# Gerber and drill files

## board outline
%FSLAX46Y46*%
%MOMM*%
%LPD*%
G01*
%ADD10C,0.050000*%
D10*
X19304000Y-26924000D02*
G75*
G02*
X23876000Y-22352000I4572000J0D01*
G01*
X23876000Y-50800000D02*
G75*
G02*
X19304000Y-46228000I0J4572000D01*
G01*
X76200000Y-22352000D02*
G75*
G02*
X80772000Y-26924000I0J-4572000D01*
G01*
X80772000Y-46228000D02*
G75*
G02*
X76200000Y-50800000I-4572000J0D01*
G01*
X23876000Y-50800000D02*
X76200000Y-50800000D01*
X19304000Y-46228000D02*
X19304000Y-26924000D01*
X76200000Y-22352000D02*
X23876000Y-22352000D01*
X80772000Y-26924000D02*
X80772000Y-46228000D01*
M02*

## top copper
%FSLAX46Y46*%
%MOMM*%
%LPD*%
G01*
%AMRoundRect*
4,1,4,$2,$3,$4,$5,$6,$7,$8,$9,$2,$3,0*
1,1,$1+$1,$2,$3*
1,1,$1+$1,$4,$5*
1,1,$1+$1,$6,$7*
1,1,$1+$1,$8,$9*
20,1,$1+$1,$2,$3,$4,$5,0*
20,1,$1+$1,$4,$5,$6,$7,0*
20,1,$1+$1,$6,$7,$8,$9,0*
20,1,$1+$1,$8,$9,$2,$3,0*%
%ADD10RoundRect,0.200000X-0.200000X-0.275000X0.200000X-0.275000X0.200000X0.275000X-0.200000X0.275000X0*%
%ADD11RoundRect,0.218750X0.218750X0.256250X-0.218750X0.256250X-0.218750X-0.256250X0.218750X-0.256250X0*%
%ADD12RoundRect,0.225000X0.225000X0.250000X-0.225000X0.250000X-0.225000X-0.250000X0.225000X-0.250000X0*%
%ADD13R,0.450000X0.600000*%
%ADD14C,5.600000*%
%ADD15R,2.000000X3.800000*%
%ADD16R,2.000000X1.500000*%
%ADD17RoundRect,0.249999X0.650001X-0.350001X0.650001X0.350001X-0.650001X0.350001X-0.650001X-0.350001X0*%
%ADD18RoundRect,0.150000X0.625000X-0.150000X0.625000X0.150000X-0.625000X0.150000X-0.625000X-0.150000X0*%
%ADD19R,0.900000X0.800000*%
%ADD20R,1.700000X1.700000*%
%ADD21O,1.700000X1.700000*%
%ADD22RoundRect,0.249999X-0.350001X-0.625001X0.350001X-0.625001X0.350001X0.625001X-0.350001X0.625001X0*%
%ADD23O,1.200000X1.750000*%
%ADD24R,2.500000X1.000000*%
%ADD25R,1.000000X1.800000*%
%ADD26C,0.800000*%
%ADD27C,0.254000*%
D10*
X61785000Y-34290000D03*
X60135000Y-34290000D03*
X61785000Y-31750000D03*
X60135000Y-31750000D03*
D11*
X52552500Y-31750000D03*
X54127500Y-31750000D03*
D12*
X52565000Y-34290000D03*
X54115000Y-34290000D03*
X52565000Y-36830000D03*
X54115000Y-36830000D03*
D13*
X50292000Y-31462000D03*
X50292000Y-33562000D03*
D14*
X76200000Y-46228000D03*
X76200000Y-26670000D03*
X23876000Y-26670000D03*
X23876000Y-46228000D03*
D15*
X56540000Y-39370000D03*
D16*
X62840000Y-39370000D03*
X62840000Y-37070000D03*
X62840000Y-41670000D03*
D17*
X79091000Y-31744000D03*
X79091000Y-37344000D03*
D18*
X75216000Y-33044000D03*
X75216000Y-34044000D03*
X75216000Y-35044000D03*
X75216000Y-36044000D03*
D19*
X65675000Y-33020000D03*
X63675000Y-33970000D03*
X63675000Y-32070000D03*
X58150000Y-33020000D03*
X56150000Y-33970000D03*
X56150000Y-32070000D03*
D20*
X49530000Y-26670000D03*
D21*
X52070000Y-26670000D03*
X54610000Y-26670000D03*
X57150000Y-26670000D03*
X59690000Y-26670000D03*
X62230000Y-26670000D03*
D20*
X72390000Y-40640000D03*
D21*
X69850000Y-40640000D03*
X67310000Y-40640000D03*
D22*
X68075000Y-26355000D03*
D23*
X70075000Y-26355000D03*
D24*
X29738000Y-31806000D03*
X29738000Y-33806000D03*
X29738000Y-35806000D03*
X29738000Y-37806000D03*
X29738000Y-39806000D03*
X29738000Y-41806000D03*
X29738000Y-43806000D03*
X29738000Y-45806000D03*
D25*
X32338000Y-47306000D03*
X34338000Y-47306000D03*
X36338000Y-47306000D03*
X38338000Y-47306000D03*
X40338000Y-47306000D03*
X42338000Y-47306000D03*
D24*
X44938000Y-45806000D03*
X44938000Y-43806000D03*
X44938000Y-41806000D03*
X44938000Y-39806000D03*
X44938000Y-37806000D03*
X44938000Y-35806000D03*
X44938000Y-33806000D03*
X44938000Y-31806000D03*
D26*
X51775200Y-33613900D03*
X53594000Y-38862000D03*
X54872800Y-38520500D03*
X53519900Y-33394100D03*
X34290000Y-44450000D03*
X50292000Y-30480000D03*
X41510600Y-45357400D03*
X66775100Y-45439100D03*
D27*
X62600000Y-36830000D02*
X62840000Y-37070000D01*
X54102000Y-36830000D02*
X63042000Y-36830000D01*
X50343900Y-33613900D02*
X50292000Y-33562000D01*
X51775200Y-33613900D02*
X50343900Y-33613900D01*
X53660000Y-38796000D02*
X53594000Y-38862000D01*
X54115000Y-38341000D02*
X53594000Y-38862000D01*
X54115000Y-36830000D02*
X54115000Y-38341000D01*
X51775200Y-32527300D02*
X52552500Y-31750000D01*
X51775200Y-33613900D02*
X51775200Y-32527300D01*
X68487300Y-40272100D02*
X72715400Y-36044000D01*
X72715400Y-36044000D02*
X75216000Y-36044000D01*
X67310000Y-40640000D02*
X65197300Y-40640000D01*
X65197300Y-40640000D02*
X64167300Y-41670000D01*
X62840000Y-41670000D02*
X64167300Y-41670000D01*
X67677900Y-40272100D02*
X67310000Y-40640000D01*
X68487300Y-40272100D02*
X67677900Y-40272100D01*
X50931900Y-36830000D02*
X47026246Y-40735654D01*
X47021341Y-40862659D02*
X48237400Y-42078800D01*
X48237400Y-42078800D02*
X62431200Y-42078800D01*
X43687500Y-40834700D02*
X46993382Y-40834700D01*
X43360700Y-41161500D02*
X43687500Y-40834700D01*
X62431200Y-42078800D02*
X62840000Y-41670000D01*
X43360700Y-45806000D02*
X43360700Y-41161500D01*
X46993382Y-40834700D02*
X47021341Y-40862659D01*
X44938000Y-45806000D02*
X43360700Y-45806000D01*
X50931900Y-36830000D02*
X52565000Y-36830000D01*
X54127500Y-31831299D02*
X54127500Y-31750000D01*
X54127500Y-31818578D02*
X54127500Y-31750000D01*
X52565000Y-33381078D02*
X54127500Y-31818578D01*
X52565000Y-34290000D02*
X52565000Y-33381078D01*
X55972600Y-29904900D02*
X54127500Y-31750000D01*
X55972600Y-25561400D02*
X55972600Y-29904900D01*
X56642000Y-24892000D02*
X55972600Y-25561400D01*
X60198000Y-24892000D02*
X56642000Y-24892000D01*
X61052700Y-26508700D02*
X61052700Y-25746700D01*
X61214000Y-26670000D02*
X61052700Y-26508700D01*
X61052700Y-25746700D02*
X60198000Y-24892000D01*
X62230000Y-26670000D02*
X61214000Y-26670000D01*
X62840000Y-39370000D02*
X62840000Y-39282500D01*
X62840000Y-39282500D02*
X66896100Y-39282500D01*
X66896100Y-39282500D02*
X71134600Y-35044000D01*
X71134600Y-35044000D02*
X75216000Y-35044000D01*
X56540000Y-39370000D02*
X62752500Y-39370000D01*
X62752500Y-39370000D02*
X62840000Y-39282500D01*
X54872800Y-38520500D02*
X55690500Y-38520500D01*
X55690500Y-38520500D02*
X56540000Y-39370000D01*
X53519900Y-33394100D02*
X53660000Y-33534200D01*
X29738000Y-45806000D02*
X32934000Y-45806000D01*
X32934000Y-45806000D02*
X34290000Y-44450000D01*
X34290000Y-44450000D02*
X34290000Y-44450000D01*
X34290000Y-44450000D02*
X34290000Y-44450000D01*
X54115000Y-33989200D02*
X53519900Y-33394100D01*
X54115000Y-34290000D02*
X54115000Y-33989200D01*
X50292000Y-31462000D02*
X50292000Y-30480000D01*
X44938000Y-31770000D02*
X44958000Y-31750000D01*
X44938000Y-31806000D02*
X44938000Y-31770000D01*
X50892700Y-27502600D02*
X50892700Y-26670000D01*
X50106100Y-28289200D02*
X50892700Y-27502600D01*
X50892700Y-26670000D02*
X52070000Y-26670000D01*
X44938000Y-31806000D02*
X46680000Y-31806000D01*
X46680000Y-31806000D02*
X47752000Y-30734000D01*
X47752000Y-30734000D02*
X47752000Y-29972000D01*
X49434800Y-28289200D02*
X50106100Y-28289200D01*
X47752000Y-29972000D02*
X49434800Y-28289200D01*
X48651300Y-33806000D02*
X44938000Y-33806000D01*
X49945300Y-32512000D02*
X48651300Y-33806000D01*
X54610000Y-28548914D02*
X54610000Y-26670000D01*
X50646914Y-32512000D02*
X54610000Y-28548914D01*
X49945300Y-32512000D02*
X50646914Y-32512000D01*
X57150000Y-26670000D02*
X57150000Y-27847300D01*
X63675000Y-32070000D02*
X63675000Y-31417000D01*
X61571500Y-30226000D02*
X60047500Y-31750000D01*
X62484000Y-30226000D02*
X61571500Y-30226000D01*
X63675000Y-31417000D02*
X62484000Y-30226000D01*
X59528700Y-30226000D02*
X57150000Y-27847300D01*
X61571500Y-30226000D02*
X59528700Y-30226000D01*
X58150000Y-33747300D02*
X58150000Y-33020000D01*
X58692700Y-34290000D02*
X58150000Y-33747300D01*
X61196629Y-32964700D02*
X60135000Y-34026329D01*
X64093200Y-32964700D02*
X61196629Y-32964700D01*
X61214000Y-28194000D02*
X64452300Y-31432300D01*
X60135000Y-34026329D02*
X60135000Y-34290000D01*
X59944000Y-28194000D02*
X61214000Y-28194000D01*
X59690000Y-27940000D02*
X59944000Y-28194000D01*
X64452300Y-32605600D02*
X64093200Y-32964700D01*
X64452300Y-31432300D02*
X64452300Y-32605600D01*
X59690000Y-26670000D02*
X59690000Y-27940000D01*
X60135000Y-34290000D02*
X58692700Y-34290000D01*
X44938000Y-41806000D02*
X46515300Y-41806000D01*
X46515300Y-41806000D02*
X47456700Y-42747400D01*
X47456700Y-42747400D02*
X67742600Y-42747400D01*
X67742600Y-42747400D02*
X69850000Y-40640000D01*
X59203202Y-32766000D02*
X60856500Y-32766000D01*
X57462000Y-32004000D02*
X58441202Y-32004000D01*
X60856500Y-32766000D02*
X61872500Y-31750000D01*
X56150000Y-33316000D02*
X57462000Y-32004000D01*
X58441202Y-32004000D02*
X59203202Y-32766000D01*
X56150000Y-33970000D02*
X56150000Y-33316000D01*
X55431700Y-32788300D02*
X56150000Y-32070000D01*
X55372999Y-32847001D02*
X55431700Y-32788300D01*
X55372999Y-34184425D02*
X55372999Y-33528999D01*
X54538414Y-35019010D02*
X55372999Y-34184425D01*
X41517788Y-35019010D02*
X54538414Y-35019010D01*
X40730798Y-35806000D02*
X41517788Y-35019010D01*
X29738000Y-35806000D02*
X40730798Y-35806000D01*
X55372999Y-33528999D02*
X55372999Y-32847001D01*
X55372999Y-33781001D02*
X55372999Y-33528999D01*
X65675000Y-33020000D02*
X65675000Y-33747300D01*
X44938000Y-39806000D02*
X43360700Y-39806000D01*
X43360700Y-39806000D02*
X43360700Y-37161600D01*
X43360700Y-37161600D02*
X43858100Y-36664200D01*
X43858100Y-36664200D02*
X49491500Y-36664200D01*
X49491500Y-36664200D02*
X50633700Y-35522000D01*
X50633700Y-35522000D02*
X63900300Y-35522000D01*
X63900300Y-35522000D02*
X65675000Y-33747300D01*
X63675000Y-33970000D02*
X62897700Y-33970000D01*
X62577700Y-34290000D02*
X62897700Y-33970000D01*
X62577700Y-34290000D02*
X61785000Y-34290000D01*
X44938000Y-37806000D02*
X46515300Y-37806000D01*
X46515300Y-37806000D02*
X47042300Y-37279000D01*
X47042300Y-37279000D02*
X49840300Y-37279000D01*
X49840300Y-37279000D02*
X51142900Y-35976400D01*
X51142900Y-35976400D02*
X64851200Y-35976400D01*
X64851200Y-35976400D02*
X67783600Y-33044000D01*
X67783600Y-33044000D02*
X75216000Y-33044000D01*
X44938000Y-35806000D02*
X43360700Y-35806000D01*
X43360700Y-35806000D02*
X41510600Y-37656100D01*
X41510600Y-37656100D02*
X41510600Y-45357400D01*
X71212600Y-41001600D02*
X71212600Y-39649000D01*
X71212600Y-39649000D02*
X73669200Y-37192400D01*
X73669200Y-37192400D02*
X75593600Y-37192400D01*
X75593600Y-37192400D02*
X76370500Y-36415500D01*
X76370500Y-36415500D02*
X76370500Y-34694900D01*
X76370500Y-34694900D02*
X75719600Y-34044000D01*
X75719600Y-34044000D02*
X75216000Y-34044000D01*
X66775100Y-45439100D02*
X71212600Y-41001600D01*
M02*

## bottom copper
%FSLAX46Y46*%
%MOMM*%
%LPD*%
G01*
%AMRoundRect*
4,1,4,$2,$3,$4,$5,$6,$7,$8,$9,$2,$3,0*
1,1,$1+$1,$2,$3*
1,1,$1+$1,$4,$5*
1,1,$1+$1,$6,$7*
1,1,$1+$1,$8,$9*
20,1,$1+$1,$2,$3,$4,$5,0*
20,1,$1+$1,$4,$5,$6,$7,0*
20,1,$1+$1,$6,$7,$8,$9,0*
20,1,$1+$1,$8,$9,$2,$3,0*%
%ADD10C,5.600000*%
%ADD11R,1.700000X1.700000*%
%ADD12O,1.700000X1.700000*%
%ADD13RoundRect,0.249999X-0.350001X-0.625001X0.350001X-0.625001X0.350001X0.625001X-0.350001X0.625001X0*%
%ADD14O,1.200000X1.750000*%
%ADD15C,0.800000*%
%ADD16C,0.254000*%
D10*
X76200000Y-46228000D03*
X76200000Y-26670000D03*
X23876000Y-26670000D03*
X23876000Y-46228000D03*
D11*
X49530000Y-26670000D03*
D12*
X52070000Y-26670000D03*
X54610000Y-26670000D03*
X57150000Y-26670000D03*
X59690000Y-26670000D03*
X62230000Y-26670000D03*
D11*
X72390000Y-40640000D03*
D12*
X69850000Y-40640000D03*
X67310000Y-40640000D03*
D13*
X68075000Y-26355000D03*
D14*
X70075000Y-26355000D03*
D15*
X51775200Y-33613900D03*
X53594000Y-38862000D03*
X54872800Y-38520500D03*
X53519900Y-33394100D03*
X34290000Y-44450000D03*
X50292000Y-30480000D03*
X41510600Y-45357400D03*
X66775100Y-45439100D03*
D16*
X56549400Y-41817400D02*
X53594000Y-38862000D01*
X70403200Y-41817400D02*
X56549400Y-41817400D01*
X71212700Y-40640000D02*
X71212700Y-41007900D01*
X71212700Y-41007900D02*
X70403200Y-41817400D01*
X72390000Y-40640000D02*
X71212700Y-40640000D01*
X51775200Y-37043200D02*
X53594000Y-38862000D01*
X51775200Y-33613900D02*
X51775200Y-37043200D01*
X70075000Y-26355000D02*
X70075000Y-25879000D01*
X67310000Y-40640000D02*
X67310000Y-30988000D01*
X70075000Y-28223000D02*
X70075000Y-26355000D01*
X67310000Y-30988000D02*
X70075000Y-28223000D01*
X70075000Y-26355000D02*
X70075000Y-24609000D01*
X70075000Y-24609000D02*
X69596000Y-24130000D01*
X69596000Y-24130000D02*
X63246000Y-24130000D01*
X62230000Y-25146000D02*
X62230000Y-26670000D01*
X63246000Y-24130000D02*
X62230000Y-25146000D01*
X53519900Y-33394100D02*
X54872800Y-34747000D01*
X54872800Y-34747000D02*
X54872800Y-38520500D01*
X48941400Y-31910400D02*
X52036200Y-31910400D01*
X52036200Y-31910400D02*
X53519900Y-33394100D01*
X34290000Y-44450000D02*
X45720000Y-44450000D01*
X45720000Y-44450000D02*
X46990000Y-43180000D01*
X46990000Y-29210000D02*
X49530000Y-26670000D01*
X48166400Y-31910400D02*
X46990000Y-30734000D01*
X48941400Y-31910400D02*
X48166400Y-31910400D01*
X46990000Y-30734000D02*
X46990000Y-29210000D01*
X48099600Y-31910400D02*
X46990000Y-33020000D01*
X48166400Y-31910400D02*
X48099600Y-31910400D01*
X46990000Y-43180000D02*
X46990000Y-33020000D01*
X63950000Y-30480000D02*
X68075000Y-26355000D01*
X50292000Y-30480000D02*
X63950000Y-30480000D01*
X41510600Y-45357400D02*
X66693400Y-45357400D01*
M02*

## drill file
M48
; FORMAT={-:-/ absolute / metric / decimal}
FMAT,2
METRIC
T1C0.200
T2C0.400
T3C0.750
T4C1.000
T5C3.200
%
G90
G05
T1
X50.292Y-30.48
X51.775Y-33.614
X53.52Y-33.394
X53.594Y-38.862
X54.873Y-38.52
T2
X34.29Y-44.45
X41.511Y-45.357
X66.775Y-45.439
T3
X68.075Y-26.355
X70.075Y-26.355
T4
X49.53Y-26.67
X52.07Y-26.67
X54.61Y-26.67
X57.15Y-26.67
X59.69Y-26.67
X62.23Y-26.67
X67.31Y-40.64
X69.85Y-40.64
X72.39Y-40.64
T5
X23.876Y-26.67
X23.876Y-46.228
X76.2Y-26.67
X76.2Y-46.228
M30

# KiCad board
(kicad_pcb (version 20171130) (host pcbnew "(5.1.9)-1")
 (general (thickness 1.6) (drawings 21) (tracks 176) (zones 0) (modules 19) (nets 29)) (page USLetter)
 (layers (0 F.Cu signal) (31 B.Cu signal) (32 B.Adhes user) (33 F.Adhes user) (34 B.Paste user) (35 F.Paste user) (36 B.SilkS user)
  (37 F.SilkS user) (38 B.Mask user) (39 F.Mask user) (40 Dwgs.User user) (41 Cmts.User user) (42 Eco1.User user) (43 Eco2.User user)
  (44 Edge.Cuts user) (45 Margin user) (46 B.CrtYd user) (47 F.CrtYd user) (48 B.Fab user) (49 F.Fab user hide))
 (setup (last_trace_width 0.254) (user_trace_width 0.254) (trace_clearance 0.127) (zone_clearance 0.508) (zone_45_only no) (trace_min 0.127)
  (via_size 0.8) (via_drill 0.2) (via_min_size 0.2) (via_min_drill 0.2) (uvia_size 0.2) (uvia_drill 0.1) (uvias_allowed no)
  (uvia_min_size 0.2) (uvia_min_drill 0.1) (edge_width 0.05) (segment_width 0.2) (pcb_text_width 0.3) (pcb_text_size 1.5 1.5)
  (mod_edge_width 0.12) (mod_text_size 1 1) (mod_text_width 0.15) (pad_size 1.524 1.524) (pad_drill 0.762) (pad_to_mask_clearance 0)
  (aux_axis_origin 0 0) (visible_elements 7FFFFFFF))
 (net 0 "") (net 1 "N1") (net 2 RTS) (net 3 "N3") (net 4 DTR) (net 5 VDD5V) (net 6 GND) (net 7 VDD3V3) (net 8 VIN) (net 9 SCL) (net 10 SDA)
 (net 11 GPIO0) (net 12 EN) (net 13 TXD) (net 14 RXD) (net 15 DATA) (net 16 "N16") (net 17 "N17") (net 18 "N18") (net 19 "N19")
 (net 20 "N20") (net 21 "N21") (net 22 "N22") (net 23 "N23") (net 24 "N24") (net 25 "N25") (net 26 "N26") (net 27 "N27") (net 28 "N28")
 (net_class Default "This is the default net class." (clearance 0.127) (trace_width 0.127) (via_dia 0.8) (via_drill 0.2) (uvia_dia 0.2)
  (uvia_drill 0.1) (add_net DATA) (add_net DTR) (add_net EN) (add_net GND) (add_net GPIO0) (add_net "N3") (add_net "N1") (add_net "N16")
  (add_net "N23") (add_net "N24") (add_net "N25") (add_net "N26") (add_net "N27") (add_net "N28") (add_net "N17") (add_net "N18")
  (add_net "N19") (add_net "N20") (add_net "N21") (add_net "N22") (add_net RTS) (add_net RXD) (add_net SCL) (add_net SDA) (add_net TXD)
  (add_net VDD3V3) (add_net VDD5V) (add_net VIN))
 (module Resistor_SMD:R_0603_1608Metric (layer F.Cu) (at 60.96 34.29)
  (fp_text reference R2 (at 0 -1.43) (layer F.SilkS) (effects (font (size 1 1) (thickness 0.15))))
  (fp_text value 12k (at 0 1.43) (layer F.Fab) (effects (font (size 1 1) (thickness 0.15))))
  (pad 2 smd roundrect (at 0.825 0) (size 0.8 0.95) (layers F.Cu F.Paste F.Mask) (roundrect_rratio 0.25) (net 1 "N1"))
  (pad 1 smd roundrect (at -0.825 0) (size 0.8 0.95) (layers F.Cu F.Paste F.Mask) (roundrect_rratio 0.25) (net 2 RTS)))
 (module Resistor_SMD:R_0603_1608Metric (layer F.Cu) (at 60.96 31.75)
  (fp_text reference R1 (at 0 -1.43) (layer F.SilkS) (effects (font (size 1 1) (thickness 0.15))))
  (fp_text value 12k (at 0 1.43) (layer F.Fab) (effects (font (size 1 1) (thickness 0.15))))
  (pad 2 smd roundrect (at 0.825 0) (size 0.8 0.95) (layers F.Cu F.Paste F.Mask) (roundrect_rratio 0.25) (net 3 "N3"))
  (pad 1 smd roundrect (at -0.825 0) (size 0.8 0.95) (layers F.Cu F.Paste F.Mask) (roundrect_rratio 0.25) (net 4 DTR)))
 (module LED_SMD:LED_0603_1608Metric (layer F.Cu) (at 53.34 31.75 180)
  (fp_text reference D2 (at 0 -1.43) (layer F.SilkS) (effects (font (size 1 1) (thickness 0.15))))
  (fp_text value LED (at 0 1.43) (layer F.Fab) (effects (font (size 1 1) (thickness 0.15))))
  (pad 2 smd roundrect (at 0.7875 0 180) (size 0.875 0.95) (layers F.Cu F.Paste F.Mask) (roundrect_rratio 0.25) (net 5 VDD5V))
  (pad 1 smd roundrect (at -0.7875 0 180) (size 0.875 0.95) (layers F.Cu F.Paste F.Mask) (roundrect_rratio 0.25) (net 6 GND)))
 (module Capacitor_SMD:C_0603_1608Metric (layer F.Cu) (at 53.34 34.29 180)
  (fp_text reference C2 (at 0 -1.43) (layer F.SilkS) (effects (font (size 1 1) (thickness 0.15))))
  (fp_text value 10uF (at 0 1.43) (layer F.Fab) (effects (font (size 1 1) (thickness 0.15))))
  (pad 2 smd roundrect (at 0.775 0 180) (size 0.9 0.95) (layers F.Cu F.Paste F.Mask) (roundrect_rratio 0.25) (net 6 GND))
  (pad 1 smd roundrect (at -0.775 0 180) (size 0.9 0.95) (layers F.Cu F.Paste F.Mask) (roundrect_rratio 0.25) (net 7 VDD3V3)))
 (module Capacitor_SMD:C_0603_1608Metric (layer F.Cu) (at 53.34 36.83 180)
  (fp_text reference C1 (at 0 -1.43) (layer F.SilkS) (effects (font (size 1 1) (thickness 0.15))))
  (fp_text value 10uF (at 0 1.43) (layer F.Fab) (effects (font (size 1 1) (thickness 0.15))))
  (pad 2 smd roundrect (at 0.775 0 180) (size 0.9 0.95) (layers F.Cu F.Paste F.Mask) (roundrect_rratio 0.25) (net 6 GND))
  (pad 1 smd roundrect (at -0.775 0 180) (size 0.9 0.95) (layers F.Cu F.Paste F.Mask) (roundrect_rratio 0.25) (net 5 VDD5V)))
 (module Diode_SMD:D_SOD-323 (layer F.Cu) (at 50.292 32.512 90)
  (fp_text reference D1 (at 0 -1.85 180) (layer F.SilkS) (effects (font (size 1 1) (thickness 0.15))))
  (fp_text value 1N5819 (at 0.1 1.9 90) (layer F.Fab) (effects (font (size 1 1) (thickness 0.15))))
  (pad 2 smd rect (at 1.05 0 90) (size 0.6 0.45) (layers F.Cu F.Paste F.Mask) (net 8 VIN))
  (pad 1 smd rect (at -1.05 0 90) (size 0.6 0.45) (layers F.Cu F.Paste F.Mask) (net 5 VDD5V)))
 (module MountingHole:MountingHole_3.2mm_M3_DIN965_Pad (layer F.Cu) (at 76.2 46.228)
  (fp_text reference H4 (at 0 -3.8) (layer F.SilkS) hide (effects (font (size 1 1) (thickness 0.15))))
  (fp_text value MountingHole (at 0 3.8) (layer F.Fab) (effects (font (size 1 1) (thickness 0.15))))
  (pad 1 thru_hole circle (at 0 0) (size 5.6 5.6) (drill 3.2) (layers *.Cu *.Mask)))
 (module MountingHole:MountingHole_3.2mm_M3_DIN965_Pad (layer F.Cu) (at 76.2 26.67)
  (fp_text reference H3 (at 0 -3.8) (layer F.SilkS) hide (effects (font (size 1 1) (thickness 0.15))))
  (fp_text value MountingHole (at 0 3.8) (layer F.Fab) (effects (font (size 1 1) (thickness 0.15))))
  (pad 1 thru_hole circle (at 0 0) (size 5.6 5.6) (drill 3.2) (layers *.Cu *.Mask)))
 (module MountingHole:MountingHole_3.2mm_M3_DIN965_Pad (layer F.Cu) (at 23.876 26.67)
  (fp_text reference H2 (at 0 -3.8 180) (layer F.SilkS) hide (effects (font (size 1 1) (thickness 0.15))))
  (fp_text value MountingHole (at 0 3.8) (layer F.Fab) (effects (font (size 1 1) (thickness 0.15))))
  (pad 1 thru_hole circle (at 0 0) (size 5.6 5.6) (drill 3.2) (layers *.Cu *.Mask)))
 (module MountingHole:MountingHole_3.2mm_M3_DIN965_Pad (layer F.Cu) (at 23.876 46.228)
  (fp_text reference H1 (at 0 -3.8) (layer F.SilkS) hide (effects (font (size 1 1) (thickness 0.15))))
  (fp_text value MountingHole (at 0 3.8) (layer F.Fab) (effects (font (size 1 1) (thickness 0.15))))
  (pad 1 thru_hole circle (at 0 0) (size 5.6 5.6) (drill 3.2) (layers *.Cu *.Mask)))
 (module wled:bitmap (layer F.Cu) (at 70.612 34.29)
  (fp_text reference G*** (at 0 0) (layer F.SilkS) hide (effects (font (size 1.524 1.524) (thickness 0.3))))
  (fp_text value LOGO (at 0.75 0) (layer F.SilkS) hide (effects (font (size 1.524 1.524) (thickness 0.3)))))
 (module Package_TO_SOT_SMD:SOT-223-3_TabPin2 (layer F.Cu) (at 59.69 39.37 180)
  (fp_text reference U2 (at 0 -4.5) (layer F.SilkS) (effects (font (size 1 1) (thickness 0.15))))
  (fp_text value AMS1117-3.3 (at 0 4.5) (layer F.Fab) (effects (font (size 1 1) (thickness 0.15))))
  (pad 2 smd rect (at 3.15 0 180) (size 2 3.8) (layers F.Cu F.Paste F.Mask) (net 7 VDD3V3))
  (pad 2 smd rect (at -3.15 0 180) (size 2 1.5) (layers F.Cu F.Paste F.Mask) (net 7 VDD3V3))
  (pad 3 smd rect (at -3.15 2.3 180) (size 2 1.5) (layers F.Cu F.Paste F.Mask) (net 5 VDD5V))
  (pad 1 smd rect (at -3.15 -2.3 180) (size 2 1.5) (layers F.Cu F.Paste F.Mask) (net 6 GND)))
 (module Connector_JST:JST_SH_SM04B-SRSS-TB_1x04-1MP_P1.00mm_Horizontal (layer F.Cu) (at 77.216 34.544 90)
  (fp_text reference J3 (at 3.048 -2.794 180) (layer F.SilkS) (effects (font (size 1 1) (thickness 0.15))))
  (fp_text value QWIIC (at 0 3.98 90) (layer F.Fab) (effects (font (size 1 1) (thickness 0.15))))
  (pad MP smd roundrect (at 2.8 1.875 90) (size 1.2 1.8) (layers F.Cu F.Paste F.Mask) (roundrect_rratio 0.2083325))
  (pad MP smd roundrect (at -2.8 1.875 90) (size 1.2 1.8) (layers F.Cu F.Paste F.Mask) (roundrect_rratio 0.2083325))
  (pad 4 smd roundrect (at 1.5 -2 90) (size 0.6 1.55) (layers F.Cu F.Paste F.Mask) (roundrect_rratio 0.25) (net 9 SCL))
  (pad 3 smd roundrect (at 0.5 -2 90) (size 0.6 1.55) (layers F.Cu F.Paste F.Mask) (roundrect_rratio 0.25) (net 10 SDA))
  (pad 2 smd roundrect (at -0.5 -2 90) (size 0.6 1.55) (layers F.Cu F.Paste F.Mask) (roundrect_rratio 0.25) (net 7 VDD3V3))
  (pad 1 smd roundrect (at -1.5 -2 90) (size 0.6 1.55) (layers F.Cu F.Paste F.Mask) (roundrect_rratio 0.25) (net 6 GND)))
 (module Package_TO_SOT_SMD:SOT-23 (layer F.Cu) (at 64.675 33.02)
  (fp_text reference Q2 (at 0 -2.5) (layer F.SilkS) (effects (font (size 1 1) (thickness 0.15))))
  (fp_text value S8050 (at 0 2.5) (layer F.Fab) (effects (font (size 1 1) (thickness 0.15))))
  (pad 3 smd rect (at 1 0) (size 0.9 0.8) (layers F.Cu F.Paste F.Mask) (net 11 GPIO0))
  (pad 2 smd rect (at -1 0.95) (size 0.9 0.8) (layers F.Cu F.Paste F.Mask) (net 1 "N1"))
  (pad 1 smd rect (at -1 -0.95) (size 0.9 0.8) (layers F.Cu F.Paste F.Mask) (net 4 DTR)))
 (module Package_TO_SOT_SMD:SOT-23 (layer F.Cu) (at 57.15 33.02)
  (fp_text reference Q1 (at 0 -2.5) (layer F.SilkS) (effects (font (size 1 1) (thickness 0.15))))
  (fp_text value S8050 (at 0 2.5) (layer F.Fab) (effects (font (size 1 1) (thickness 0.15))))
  (pad 3 smd rect (at 1 0) (size 0.9 0.8) (layers F.Cu F.Paste F.Mask) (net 2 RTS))
  (pad 2 smd rect (at -1 0.95) (size 0.9 0.8) (layers F.Cu F.Paste F.Mask) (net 3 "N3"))
  (pad 1 smd rect (at -1 -0.95) (size 0.9 0.8) (layers F.Cu F.Paste F.Mask) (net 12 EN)))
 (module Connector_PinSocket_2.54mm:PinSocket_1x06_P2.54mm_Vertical (layer F.Cu) (at 49.53 26.67 90)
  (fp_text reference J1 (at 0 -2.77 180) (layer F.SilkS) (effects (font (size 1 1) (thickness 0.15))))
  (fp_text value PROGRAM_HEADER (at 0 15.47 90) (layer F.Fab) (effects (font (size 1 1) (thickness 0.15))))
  (pad 1 thru_hole rect (at 0 0 90) (size 1.7 1.7) (drill 1) (layers *.Cu *.Mask) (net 7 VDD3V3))
  (pad 2 thru_hole oval (at 0 2.54 90) (size 1.7 1.7) (drill 1) (layers *.Cu *.Mask) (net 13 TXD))
  (pad 3 thru_hole oval (at 0 5.08 90) (size 1.7 1.7) (drill 1) (layers *.Cu *.Mask) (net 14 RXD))
  (pad 4 thru_hole oval (at 0 7.62 90) (size 1.7 1.7) (drill 1) (layers *.Cu *.Mask) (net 4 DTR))
  (pad 5 thru_hole oval (at 0 10.16 90) (size 1.7 1.7) (drill 1) (layers *.Cu *.Mask) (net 2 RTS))
  (pad 6 thru_hole oval (at 0 12.7 90) (size 1.7 1.7) (drill 1) (layers *.Cu *.Mask) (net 6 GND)))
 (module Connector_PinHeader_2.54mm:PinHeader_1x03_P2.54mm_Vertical (layer F.Cu) (at 72.39 40.64 270)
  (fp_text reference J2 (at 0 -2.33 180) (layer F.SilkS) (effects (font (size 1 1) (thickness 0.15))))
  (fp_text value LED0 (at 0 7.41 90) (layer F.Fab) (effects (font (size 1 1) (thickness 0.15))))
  (pad 1 thru_hole rect (at 0 0 270) (size 1.7 1.7) (drill 1) (layers *.Cu *.Mask) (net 5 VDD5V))
  (pad 2 thru_hole oval (at 0 2.54 270) (size 1.7 1.7) (drill 1) (layers *.Cu *.Mask) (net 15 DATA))
  (pad 3 thru_hole oval (at 0 5.08 270) (size 1.7 1.7) (drill 1) (layers *.Cu *.Mask) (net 6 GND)))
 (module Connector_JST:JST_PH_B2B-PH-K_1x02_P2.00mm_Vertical (layer F.Cu) (at 68.075 26.355)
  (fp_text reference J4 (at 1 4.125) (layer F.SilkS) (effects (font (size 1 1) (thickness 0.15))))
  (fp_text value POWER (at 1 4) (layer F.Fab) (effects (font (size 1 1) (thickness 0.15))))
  (pad 1 thru_hole roundrect (at 0 0) (size 1.2 1.75) (drill 0.75) (layers *.Cu *.Mask) (roundrect_rratio 0.2083325) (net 8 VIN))
  (pad 2 thru_hole oval (at 2 0) (size 1.2 1.75) (drill 0.75) (layers *.Cu *.Mask) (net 6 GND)))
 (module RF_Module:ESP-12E (layer F.Cu) (at 37.338 35.306)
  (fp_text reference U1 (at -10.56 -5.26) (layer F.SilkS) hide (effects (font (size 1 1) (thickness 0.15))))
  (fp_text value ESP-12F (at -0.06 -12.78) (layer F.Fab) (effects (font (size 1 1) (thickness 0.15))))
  (pad 1 smd rect (at -7.6 -3.5) (size 2.5 1) (layers F.Cu F.Paste F.Mask) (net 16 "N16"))
  (pad 2 smd rect (at -7.6 -1.5) (size 2.5 1) (layers F.Cu F.Paste F.Mask) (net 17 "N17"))
  (pad 3 smd rect (at -7.6 0.5) (size 2.5 1) (layers F.Cu F.Paste F.Mask) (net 12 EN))
  (pad 4 smd rect (at -7.6 2.5) (size 2.5 1) (layers F.Cu F.Paste F.Mask) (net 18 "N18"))
  (pad 5 smd rect (at -7.6 4.5) (size 2.5 1) (layers F.Cu F.Paste F.Mask) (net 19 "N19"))
  (pad 6 smd rect (at -7.6 6.5) (size 2.5 1) (layers F.Cu F.Paste F.Mask) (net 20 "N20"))
  (pad 7 smd rect (at -7.6 8.5) (size 2.5 1) (layers F.Cu F.Paste F.Mask) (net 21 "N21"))
  (pad 8 smd rect (at -7.6 10.5) (size 2.5 1) (layers F.Cu F.Paste F.Mask) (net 7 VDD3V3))
  (pad 9 smd rect (at -5 12) (size 1 1.8) (layers F.Cu F.Paste F.Mask) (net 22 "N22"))
  (pad 10 smd rect (at -3 12) (size 1 1.8) (layers F.Cu F.Paste F.Mask) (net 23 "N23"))
  (pad 11 smd rect (at -1 12) (size 1 1.8) (layers F.Cu F.Paste F.Mask) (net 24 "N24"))
  (pad 12 smd rect (at 1 12) (size 1 1.8) (layers F.Cu F.Paste F.Mask) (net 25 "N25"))
  (pad 13 smd rect (at 3 12) (size 1 1.8) (layers F.Cu F.Paste F.Mask) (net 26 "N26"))
  (pad 14 smd rect (at 5 12) (size 1 1.8) (layers F.Cu F.Paste F.Mask) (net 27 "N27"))
  (pad 15 smd rect (at 7.6 10.5) (size 2.5 1) (layers F.Cu F.Paste F.Mask) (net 6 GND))
  (pad 16 smd rect (at 7.6 8.5) (size 2.5 1) (layers F.Cu F.Paste F.Mask) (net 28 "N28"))
  (pad 17 smd rect (at 7.6 6.5) (size 2.5 1) (layers F.Cu F.Paste F.Mask) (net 15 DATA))
  (pad 18 smd rect (at 7.6 4.5) (size 2.5 1) (layers F.Cu F.Paste F.Mask) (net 11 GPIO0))
  (pad 19 smd rect (at 7.6 2.5) (size 2.5 1) (layers F.Cu F.Paste F.Mask) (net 9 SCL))
  (pad 20 smd rect (at 7.6 0.5) (size 2.5 1) (layers F.Cu F.Paste F.Mask) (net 10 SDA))
  (pad 21 smd rect (at 7.6 -1.5) (size 2.5 1) (layers F.Cu F.Paste F.Mask) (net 14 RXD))
  (pad 22 smd rect (at 7.6 -3.5) (size 2.5 1) (layers F.Cu F.Paste F.Mask) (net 13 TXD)))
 (gr_arc (start 23.876 26.924) (end 23.876 22.352) (angle -90) (layer Edge.Cuts) (width 0.05))
 (gr_arc (start 23.876 46.228) (end 19.304 46.228) (angle -90) (layer Edge.Cuts) (width 0.05))
 (gr_arc (start 76.2 26.924) (end 80.772 26.924) (angle -90) (layer Edge.Cuts) (width 0.05))
 (gr_arc (start 76.2 46.228) (end 76.2 50.8) (angle -90) (layer Edge.Cuts) (width 0.05))
 (gr_line (start 23.876 50.8) (end 76.2 50.8) (layer Edge.Cuts) (width 0.05))
 (gr_line (start 19.304 46.228) (end 19.304 26.924) (layer Edge.Cuts) (width 0.05))
 (gr_line (start 76.2 22.352) (end 23.876 22.352) (layer Edge.Cuts) (width 0.05))
 (gr_line (start 80.772 26.924) (end 80.772 46.228) (layer Edge.Cuts) (width 0.05))
 (via (at 51.7752 33.6139) (size 0.8) (layers F.Cu B.Cu) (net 5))
 (via (at 53.594 38.862) (size 0.8) (drill 0.2) (layers F.Cu B.Cu) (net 5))
 (segment (start 62.6 36.83) (end 62.84 37.07) (width 0.254) (layer F.Cu) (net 5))
 (segment (start 54.102 36.83) (end 63.042 36.83) (width 0.254) (layer F.Cu) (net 5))
 (segment (start 50.3439 33.6139) (end 50.292 33.562) (width 0.254) (layer F.Cu) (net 5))
 (segment (start 51.7752 33.6139) (end 50.3439 33.6139) (width 0.254) (layer F.Cu) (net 5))
 (segment (start 56.5494 41.8174) (end 53.594 38.862) (width 0.254) (layer B.Cu) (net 5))
 (segment (start 70.4032 41.8174) (end 56.5494 41.8174) (width 0.254) (layer B.Cu) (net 5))
 (segment (start 71.2127 40.64) (end 71.2127 41.0079) (width 0.254) (layer B.Cu) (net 5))
 (segment (start 71.2127 41.0079) (end 70.4032 41.8174) (width 0.254) (layer B.Cu) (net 5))
 (segment (start 72.39 40.64) (end 71.2127 40.64) (width 0.254) (layer B.Cu) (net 5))
 (segment (start 53.66 38.796) (end 53.594 38.862) (width 0.254) (layer F.Cu) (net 5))
 (segment (start 51.7752 37.0432) (end 53.594 38.862) (width 0.254) (layer B.Cu) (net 5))
 (segment (start 51.7752 33.6139) (end 51.7752 37.0432) (width 0.254) (layer B.Cu) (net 5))
 (segment (start 54.115 38.341) (end 53.594 38.862) (width 0.254) (layer F.Cu) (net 5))
 (segment (start 54.115 36.83) (end 54.115 38.341) (width 0.254) (layer F.Cu) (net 5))
 (segment (start 51.7752 32.5273) (end 52.5525 31.75) (width 0.254) (layer F.Cu) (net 5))
 (segment (start 51.7752 33.6139) (end 51.7752 32.5273) (width 0.254) (layer F.Cu) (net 5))
 (segment (start 68.4873 40.2721) (end 72.7154 36.044) (width 0.254) (layer F.Cu) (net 6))
 (segment (start 72.7154 36.044) (end 75.216 36.044) (width 0.254) (layer F.Cu) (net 6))
 (segment (start 67.31 40.64) (end 65.1973 40.64) (width 0.254) (layer F.Cu) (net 6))
 (segment (start 65.1973 40.64) (end 64.1673 41.67) (width 0.254) (layer F.Cu) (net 6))
 (segment (start 62.84 41.67) (end 64.1673 41.67) (width 0.254) (layer F.Cu) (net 6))
 (segment (start 70.075 26.355) (end 70.075 25.879) (width 0.254) (layer B.Cu) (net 6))
 (segment (start 67.31 40.64) (end 67.31 30.988) (width 0.254) (layer B.Cu) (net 6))
 (segment (start 70.075 28.223) (end 70.075 26.355) (width 0.254) (layer B.Cu) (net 6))
 (segment (start 67.31 30.988) (end 70.075 28.223) (width 0.254) (layer B.Cu) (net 6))
 (segment (start 70.075 26.355) (end 70.075 24.609) (width 0.254) (layer B.Cu) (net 6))
 (segment (start 70.075 24.609) (end 69.596 24.13) (width 0.254) (layer B.Cu) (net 6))
 (segment (start 69.596 24.13) (end 63.246 24.13) (width 0.254) (layer B.Cu) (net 6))
 (segment (start 62.23 25.146) (end 62.23 26.67) (width 0.254) (layer B.Cu) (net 6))
 (segment (start 63.246 24.13) (end 62.23 25.146) (width 0.254) (layer B.Cu) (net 6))
 (segment (start 67.6779 40.2721) (end 67.31 40.64) (width 0.254) (layer F.Cu) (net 6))
 (segment (start 68.4873 40.2721) (end 67.6779 40.2721) (width 0.254) (layer F.Cu) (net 6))
 (segment (start 50.9319 36.83) (end 47.026246 40.735654) (width 0.254) (layer F.Cu) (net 6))
 (segment (start 47.021341 40.862659) (end 48.2374 42.0788) (width 0.254) (layer F.Cu) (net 6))
 (segment (start 48.2374 42.0788) (end 62.4312 42.0788) (width 0.254) (layer F.Cu) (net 6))
 (segment (start 43.6875 40.8347) (end 46.993382 40.8347) (width 0.254) (layer F.Cu) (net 6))
 (segment (start 43.3607 41.1615) (end 43.6875 40.8347) (width 0.254) (layer F.Cu) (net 6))
 (segment (start 62.4312 42.0788) (end 62.84 41.67) (width 0.254) (layer F.Cu) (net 6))
 (segment (start 43.3607 45.806) (end 43.3607 41.1615) (width 0.254) (layer F.Cu) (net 6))
 (segment (start 46.993382 40.8347) (end 47.021341 40.862659) (width 0.254) (layer F.Cu) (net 6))
 (segment (start 44.938 45.806) (end 43.3607 45.806) (width 0.254) (layer F.Cu) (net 6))
 (segment (start 50.9319 36.83) (end 52.565 36.83) (width 0.254) (layer F.Cu) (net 6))
 (segment (start 54.1275 31.831299) (end 54.1275 31.75) (width 0.254) (layer F.Cu) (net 6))
 (segment (start 54.1275 31.818578) (end 54.1275 31.75) (width 0.254) (layer F.Cu) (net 6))
 (segment (start 52.565 33.381078) (end 54.1275 31.818578) (width 0.254) (layer F.Cu) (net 6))
 (segment (start 52.565 34.29) (end 52.565 33.381078) (width 0.254) (layer F.Cu) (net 6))
 (segment (start 55.9726 29.9049) (end 54.1275 31.75) (width 0.254) (layer F.Cu) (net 6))
 (segment (start 55.9726 25.5614) (end 55.9726 29.9049) (width 0.254) (layer F.Cu) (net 6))
 (segment (start 56.642 24.892) (end 55.9726 25.5614) (width 0.254) (layer F.Cu) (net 6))
 (segment (start 60.198 24.892) (end 56.642 24.892) (width 0.254) (layer F.Cu) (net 6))
 (segment (start 61.0527 26.5087) (end 61.0527 25.7467) (width 0.254) (layer F.Cu) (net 6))
 (segment (start 61.214 26.67) (end 61.0527 26.5087) (width 0.254) (layer F.Cu) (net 6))
 (segment (start 61.0527 25.7467) (end 60.198 24.892) (width 0.254) (layer F.Cu) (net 6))
 (segment (start 62.23 26.67) (end 61.214 26.67) (width 0.254) (layer F.Cu) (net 6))
 (segment (start 62.84 39.37) (end 62.84 39.2825) (width 0.254) (layer F.Cu) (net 7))
 (segment (start 62.84 39.2825) (end 66.8961 39.2825) (width 0.254) (layer F.Cu) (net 7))
 (segment (start 66.8961 39.2825) (end 71.1346 35.044) (width 0.254) (layer F.Cu) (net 7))
 (segment (start 71.1346 35.044) (end 75.216 35.044) (width 0.254) (layer F.Cu) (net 7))
 (segment (start 56.54 39.37) (end 62.7525 39.37) (width 0.254) (layer F.Cu) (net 7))
 (segment (start 62.7525 39.37) (end 62.84 39.2825) (width 0.254) (layer F.Cu) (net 7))
 (segment (start 54.8728 38.5205) (end 55.6905 38.5205) (width 0.254) (layer F.Cu) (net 7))
 (segment (start 55.6905 38.5205) (end 56.54 39.37) (width 0.254) (layer F.Cu) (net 7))
 (segment (start 53.5199 33.3941) (end 54.8728 34.747) (width 0.254) (layer B.Cu) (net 7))
 (segment (start 54.8728 34.747) (end 54.8728 38.5205) (width 0.254) (layer B.Cu) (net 7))
 (segment (start 53.5199 33.3941) (end 53.66 33.5342) (width 0.254) (layer F.Cu) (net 7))
 (segment (start 48.9414 31.9104) (end 52.0362 31.9104) (width 0.254) (layer B.Cu) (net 7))
 (segment (start 52.0362 31.9104) (end 53.5199 33.3941) (width 0.254) (layer B.Cu) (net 7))
 (via (at 54.8728 38.5205) (size 0.8) (layers F.Cu B.Cu) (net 7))
 (via (at 53.5199 33.3941) (size 0.8) (layers F.Cu B.Cu) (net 7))
 (segment (start 29.738 45.806) (end 32.934 45.806) (width 0.254) (layer F.Cu) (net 7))
 (segment (start 32.934 45.806) (end 34.29 44.45) (width 0.254) (layer F.Cu) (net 7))
 (segment (start 34.29 44.45) (end 34.29 44.45) (width 0.254) (layer F.Cu) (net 7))
 (segment (start 34.29 44.45) (end 34.29 44.45) (width 0.254) (layer F.Cu) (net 7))
 (via (at 34.29 44.45) (size 0.8) (drill 0.4) (layers F.Cu B.Cu) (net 7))
 (segment (start 34.29 44.45) (end 45.72 44.45) (width 0.254) (layer B.Cu) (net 7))
 (segment (start 45.72 44.45) (end 46.99 43.18) (width 0.254) (layer B.Cu) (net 7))
 (segment (start 46.99 29.21) (end 49.53 26.67) (width 0.254) (layer B.Cu) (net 7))
 (segment (start 48.1664 31.9104) (end 46.99 30.734) (width 0.254) (layer B.Cu) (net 7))
 (segment (start 48.9414 31.9104) (end 48.1664 31.9104) (width 0.254) (layer B.Cu) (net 7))
 (segment (start 46.99 30.734) (end 46.99 29.21) (width 0.254) (layer B.Cu) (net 7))
 (segment (start 48.0996 31.9104) (end 46.99 33.02) (width 0.254) (layer B.Cu) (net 7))
 (segment (start 48.1664 31.9104) (end 48.0996 31.9104) (width 0.254) (layer B.Cu) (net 7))
 (segment (start 46.99 43.18) (end 46.99 33.02) (width 0.254) (layer B.Cu) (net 7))
 (segment (start 54.115 33.9892) (end 53.5199 33.3941) (width 0.254) (layer F.Cu) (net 7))
 (segment (start 54.115 34.29) (end 54.115 33.9892) (width 0.254) (layer F.Cu) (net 7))
 (via (at 50.292 30.48) (size 0.8) (drill 0.2) (layers F.Cu B.Cu) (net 8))
 (segment (start 50.292 31.462) (end 50.292 30.48) (width 0.254) (layer F.Cu) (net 8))
 (segment (start 63.95 30.48) (end 68.075 26.355) (width 0.254) (layer B.Cu) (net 8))
 (segment (start 50.292 30.48) (end 63.95 30.48) (width 0.254) (layer B.Cu) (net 8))
 (segment (start 44.938 31.77) (end 44.958 31.75) (width 0.254) (layer F.Cu) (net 13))
 (segment (start 44.938 31.806) (end 44.938 31.77) (width 0.254) (layer F.Cu) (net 13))
 (segment (start 50.8927 27.5026) (end 50.8927 26.67) (width 0.254) (layer F.Cu) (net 13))
 (segment (start 50.1061 28.2892) (end 50.8927 27.5026) (width 0.254) (layer F.Cu) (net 13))
 (segment (start 50.8927 26.67) (end 52.07 26.67) (width 0.254) (layer F.Cu) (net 13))
 (segment (start 44.938 31.806) (end 46.68 31.806) (width 0.254) (layer F.Cu) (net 13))
 (segment (start 46.68 31.806) (end 47.752 30.734) (width 0.254) (layer F.Cu) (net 13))
 (segment (start 47.752 30.734) (end 47.752 29.972) (width 0.254) (layer F.Cu) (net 13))
 (segment (start 49.4348 28.2892) (end 50.1061 28.2892) (width 0.254) (layer F.Cu) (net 13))
 (segment (start 47.752 29.972) (end 49.4348 28.2892) (width 0.254) (layer F.Cu) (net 13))
 (segment (start 48.6513 33.806) (end 44.938 33.806) (width 0.254) (layer F.Cu) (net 14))
 (segment (start 49.9453 32.512) (end 48.6513 33.806) (width 0.254) (layer F.Cu) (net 14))
 (segment (start 54.61 28.548914) (end 54.61 26.67) (width 0.254) (layer F.Cu) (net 14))
 (segment (start 50.646914 32.512) (end 54.61 28.548914) (width 0.254) (layer F.Cu) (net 14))
 (segment (start 49.9453 32.512) (end 50.646914 32.512) (width 0.254) (layer F.Cu) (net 14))
 (segment (start 57.15 26.67) (end 57.15 27.8473) (width 0.254) (layer F.Cu) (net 4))
 (segment (start 63.675 32.07) (end 63.675 31.417) (width 0.254) (layer F.Cu) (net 4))
 (segment (start 61.5715 30.226) (end 60.0475 31.75) (width 0.254) (layer F.Cu) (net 4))
 (segment (start 62.484 30.226) (end 61.5715 30.226) (width 0.254) (layer F.Cu) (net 4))
 (segment (start 63.675 31.417) (end 62.484 30.226) (width 0.254) (layer F.Cu) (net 4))
 (segment (start 59.5287 30.226) (end 57.15 27.8473) (width 0.254) (layer F.Cu) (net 4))
 (segment (start 61.5715 30.226) (end 59.5287 30.226) (width 0.254) (layer F.Cu) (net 4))
 (segment (start 58.15 33.7473) (end 58.15 33.02) (width 0.254) (layer F.Cu) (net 2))
 (segment (start 58.6927 34.29) (end 58.15 33.7473) (width 0.254) (layer F.Cu) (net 2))
 (segment (start 61.196629 32.9647) (end 60.135 34.026329) (width 0.254) (layer F.Cu) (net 2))
 (segment (start 64.0932 32.9647) (end 61.196629 32.9647) (width 0.254) (layer F.Cu) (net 2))
 (segment (start 61.214 28.194) (end 64.4523 31.4323) (width 0.254) (layer F.Cu) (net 2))
 (segment (start 60.135 34.026329) (end 60.135 34.29) (width 0.254) (layer F.Cu) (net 2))
 (segment (start 59.944 28.194) (end 61.214 28.194) (width 0.254) (layer F.Cu) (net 2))
 (segment (start 59.69 27.94) (end 59.944 28.194) (width 0.254) (layer F.Cu) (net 2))
 (segment (start 64.4523 32.6056) (end 64.0932 32.9647) (width 0.254) (layer F.Cu) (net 2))
 (segment (start 64.4523 31.4323) (end 64.4523 32.6056) (width 0.254) (layer F.Cu) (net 2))
 (segment (start 59.69 26.67) (end 59.69 27.94) (width 0.254) (layer F.Cu) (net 2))
 (segment (start 60.135 34.29) (end 58.6927 34.29) (width 0.254) (layer F.Cu) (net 2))
 (segment (start 44.938 41.806) (end 46.5153 41.806) (width 0.254) (layer F.Cu) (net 15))
 (segment (start 46.5153 41.806) (end 47.4567 42.7474) (width 0.254) (layer F.Cu) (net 15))
 (segment (start 47.4567 42.7474) (end 67.7426 42.7474) (width 0.254) (layer F.Cu) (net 15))
 (segment (start 67.7426 42.7474) (end 69.85 40.64) (width 0.254) (layer F.Cu) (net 15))
 (segment (start 59.203202 32.766) (end 60.8565 32.766) (width 0.254) (layer F.Cu) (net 3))
 (segment (start 57.462 32.004) (end 58.441202 32.004) (width 0.254) (layer F.Cu) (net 3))
 (segment (start 60.8565 32.766) (end 61.8725 31.75) (width 0.254) (layer F.Cu) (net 3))
 (segment (start 56.15 33.316) (end 57.462 32.004) (width 0.254) (layer F.Cu) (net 3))
 (segment (start 58.441202 32.004) (end 59.203202 32.766) (width 0.254) (layer F.Cu) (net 3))
 (segment (start 56.15 33.97) (end 56.15 33.316) (width 0.254) (layer F.Cu) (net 3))
 (segment (start 55.4317 32.7883) (end 56.15 32.07) (width 0.254) (layer F.Cu) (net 12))
 (segment (start 55.372999 32.847001) (end 55.4317 32.7883) (width 0.254) (layer F.Cu) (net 12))
 (segment (start 55.372999 34.184425) (end 55.372999 33.528999) (width 0.254) (layer F.Cu) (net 12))
 (segment (start 54.538414 35.01901) (end 55.372999 34.184425) (width 0.254) (layer F.Cu) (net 12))
 (segment (start 41.517788 35.01901) (end 54.538414 35.01901) (width 0.254) (layer F.Cu) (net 12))
 (segment (start 40.730798 35.806) (end 41.517788 35.01901) (width 0.254) (layer F.Cu) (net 12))
 (segment (start 29.738 35.806) (end 40.730798 35.806) (width 0.254) (layer F.Cu) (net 12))
 (segment (start 55.372999 33.528999) (end 55.372999 32.847001) (width 0.254) (layer F.Cu) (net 12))
 (segment (start 55.372999 33.781001) (end 55.372999 33.528999) (width 0.254) (layer F.Cu) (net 12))
 (segment (start 65.675 33.02) (end 65.675 33.7473) (width 0.254) (layer F.Cu) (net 11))
 (segment (start 44.938 39.806) (end 43.3607 39.806) (width 0.254) (layer F.Cu) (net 11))
 (segment (start 43.3607 39.806) (end 43.3607 37.1616) (width 0.254) (layer F.Cu) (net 11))
 (segment (start 43.3607 37.1616) (end 43.8581 36.6642) (width 0.254) (layer F.Cu) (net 11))
 (segment (start 43.8581 36.6642) (end 49.4915 36.6642) (width 0.254) (layer F.Cu) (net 11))
 (segment (start 49.4915 36.6642) (end 50.6337 35.522) (width 0.254) (layer F.Cu) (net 11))
 (segment (start 50.6337 35.522) (end 63.9003 35.522) (width 0.254) (layer F.Cu) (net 11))
 (segment (start 63.9003 35.522) (end 65.675 33.7473) (width 0.254) (layer F.Cu) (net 11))
 (segment (start 63.675 33.97) (end 62.8977 33.97) (width 0.254) (layer F.Cu) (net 1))
 (segment (start 62.5777 34.29) (end 62.8977 33.97) (width 0.254) (layer F.Cu) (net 1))
 (segment (start 62.5777 34.29) (end 61.785 34.29) (width 0.254) (layer F.Cu) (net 1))
 (segment (start 44.938 37.806) (end 46.5153 37.806) (width 0.254) (layer F.Cu) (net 9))
 (segment (start 46.5153 37.806) (end 47.0423 37.279) (width 0.254) (layer F.Cu) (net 9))
 (segment (start 47.0423 37.279) (end 49.8403 37.279) (width 0.254) (layer F.Cu) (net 9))
 (segment (start 49.8403 37.279) (end 51.1429 35.9764) (width 0.254) (layer F.Cu) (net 9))
 (segment (start 51.1429 35.9764) (end 64.8512 35.9764) (width 0.254) (layer F.Cu) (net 9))
 (segment (start 64.8512 35.9764) (end 67.7836 33.044) (width 0.254) (layer F.Cu) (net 9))
 (segment (start 67.7836 33.044) (end 75.216 33.044) (width 0.254) (layer F.Cu) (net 9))
 (segment (start 44.938 35.806) (end 43.3607 35.806) (width 0.254) (layer F.Cu) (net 10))
 (segment (start 43.3607 35.806) (end 41.5106 37.6561) (width 0.254) (layer F.Cu) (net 10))
 (segment (start 41.5106 37.6561) (end 41.5106 45.3574) (width 0.254) (layer F.Cu) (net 10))
 (segment (start 71.2126 41.0016) (end 71.2126 39.649) (width 0.254) (layer F.Cu) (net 10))
 (segment (start 71.2126 39.649) (end 73.6692 37.1924) (width 0.254) (layer F.Cu) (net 10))
 (segment (start 73.6692 37.1924) (end 75.5936 37.1924) (width 0.254) (layer F.Cu) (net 10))
 (segment (start 75.5936 37.1924) (end 76.3705 36.4155) (width 0.254) (layer F.Cu) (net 10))
 (segment (start 76.3705 36.4155) (end 76.3705 34.6949) (width 0.254) (layer F.Cu) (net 10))
 (segment (start 76.3705 34.6949) (end 75.7196 34.044) (width 0.254) (layer F.Cu) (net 10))
 (segment (start 75.7196 34.044) (end 75.216 34.044) (width 0.254) (layer F.Cu) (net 10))
 (via (at 41.5106 45.3574) (size 0.8) (drill 0.4) (layers F.Cu B.Cu) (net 10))
 (segment (start 41.5106 45.3574) (end 66.6934 45.3574) (width 0.254) (layer B.Cu) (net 10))
 (segment (start 66.7751 45.4391) (end 71.2126 41.0016) (width 0.254) (layer F.Cu) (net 10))
 (via (at 66.7751 45.4391) (size 0.8) (drill 0.4) (layers F.Cu B.Cu) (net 10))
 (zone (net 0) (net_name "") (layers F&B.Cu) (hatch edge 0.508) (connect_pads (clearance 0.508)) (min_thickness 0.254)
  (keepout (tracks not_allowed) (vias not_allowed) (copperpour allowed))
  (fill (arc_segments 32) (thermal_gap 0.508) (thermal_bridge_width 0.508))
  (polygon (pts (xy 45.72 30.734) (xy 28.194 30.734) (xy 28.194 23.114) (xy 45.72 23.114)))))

